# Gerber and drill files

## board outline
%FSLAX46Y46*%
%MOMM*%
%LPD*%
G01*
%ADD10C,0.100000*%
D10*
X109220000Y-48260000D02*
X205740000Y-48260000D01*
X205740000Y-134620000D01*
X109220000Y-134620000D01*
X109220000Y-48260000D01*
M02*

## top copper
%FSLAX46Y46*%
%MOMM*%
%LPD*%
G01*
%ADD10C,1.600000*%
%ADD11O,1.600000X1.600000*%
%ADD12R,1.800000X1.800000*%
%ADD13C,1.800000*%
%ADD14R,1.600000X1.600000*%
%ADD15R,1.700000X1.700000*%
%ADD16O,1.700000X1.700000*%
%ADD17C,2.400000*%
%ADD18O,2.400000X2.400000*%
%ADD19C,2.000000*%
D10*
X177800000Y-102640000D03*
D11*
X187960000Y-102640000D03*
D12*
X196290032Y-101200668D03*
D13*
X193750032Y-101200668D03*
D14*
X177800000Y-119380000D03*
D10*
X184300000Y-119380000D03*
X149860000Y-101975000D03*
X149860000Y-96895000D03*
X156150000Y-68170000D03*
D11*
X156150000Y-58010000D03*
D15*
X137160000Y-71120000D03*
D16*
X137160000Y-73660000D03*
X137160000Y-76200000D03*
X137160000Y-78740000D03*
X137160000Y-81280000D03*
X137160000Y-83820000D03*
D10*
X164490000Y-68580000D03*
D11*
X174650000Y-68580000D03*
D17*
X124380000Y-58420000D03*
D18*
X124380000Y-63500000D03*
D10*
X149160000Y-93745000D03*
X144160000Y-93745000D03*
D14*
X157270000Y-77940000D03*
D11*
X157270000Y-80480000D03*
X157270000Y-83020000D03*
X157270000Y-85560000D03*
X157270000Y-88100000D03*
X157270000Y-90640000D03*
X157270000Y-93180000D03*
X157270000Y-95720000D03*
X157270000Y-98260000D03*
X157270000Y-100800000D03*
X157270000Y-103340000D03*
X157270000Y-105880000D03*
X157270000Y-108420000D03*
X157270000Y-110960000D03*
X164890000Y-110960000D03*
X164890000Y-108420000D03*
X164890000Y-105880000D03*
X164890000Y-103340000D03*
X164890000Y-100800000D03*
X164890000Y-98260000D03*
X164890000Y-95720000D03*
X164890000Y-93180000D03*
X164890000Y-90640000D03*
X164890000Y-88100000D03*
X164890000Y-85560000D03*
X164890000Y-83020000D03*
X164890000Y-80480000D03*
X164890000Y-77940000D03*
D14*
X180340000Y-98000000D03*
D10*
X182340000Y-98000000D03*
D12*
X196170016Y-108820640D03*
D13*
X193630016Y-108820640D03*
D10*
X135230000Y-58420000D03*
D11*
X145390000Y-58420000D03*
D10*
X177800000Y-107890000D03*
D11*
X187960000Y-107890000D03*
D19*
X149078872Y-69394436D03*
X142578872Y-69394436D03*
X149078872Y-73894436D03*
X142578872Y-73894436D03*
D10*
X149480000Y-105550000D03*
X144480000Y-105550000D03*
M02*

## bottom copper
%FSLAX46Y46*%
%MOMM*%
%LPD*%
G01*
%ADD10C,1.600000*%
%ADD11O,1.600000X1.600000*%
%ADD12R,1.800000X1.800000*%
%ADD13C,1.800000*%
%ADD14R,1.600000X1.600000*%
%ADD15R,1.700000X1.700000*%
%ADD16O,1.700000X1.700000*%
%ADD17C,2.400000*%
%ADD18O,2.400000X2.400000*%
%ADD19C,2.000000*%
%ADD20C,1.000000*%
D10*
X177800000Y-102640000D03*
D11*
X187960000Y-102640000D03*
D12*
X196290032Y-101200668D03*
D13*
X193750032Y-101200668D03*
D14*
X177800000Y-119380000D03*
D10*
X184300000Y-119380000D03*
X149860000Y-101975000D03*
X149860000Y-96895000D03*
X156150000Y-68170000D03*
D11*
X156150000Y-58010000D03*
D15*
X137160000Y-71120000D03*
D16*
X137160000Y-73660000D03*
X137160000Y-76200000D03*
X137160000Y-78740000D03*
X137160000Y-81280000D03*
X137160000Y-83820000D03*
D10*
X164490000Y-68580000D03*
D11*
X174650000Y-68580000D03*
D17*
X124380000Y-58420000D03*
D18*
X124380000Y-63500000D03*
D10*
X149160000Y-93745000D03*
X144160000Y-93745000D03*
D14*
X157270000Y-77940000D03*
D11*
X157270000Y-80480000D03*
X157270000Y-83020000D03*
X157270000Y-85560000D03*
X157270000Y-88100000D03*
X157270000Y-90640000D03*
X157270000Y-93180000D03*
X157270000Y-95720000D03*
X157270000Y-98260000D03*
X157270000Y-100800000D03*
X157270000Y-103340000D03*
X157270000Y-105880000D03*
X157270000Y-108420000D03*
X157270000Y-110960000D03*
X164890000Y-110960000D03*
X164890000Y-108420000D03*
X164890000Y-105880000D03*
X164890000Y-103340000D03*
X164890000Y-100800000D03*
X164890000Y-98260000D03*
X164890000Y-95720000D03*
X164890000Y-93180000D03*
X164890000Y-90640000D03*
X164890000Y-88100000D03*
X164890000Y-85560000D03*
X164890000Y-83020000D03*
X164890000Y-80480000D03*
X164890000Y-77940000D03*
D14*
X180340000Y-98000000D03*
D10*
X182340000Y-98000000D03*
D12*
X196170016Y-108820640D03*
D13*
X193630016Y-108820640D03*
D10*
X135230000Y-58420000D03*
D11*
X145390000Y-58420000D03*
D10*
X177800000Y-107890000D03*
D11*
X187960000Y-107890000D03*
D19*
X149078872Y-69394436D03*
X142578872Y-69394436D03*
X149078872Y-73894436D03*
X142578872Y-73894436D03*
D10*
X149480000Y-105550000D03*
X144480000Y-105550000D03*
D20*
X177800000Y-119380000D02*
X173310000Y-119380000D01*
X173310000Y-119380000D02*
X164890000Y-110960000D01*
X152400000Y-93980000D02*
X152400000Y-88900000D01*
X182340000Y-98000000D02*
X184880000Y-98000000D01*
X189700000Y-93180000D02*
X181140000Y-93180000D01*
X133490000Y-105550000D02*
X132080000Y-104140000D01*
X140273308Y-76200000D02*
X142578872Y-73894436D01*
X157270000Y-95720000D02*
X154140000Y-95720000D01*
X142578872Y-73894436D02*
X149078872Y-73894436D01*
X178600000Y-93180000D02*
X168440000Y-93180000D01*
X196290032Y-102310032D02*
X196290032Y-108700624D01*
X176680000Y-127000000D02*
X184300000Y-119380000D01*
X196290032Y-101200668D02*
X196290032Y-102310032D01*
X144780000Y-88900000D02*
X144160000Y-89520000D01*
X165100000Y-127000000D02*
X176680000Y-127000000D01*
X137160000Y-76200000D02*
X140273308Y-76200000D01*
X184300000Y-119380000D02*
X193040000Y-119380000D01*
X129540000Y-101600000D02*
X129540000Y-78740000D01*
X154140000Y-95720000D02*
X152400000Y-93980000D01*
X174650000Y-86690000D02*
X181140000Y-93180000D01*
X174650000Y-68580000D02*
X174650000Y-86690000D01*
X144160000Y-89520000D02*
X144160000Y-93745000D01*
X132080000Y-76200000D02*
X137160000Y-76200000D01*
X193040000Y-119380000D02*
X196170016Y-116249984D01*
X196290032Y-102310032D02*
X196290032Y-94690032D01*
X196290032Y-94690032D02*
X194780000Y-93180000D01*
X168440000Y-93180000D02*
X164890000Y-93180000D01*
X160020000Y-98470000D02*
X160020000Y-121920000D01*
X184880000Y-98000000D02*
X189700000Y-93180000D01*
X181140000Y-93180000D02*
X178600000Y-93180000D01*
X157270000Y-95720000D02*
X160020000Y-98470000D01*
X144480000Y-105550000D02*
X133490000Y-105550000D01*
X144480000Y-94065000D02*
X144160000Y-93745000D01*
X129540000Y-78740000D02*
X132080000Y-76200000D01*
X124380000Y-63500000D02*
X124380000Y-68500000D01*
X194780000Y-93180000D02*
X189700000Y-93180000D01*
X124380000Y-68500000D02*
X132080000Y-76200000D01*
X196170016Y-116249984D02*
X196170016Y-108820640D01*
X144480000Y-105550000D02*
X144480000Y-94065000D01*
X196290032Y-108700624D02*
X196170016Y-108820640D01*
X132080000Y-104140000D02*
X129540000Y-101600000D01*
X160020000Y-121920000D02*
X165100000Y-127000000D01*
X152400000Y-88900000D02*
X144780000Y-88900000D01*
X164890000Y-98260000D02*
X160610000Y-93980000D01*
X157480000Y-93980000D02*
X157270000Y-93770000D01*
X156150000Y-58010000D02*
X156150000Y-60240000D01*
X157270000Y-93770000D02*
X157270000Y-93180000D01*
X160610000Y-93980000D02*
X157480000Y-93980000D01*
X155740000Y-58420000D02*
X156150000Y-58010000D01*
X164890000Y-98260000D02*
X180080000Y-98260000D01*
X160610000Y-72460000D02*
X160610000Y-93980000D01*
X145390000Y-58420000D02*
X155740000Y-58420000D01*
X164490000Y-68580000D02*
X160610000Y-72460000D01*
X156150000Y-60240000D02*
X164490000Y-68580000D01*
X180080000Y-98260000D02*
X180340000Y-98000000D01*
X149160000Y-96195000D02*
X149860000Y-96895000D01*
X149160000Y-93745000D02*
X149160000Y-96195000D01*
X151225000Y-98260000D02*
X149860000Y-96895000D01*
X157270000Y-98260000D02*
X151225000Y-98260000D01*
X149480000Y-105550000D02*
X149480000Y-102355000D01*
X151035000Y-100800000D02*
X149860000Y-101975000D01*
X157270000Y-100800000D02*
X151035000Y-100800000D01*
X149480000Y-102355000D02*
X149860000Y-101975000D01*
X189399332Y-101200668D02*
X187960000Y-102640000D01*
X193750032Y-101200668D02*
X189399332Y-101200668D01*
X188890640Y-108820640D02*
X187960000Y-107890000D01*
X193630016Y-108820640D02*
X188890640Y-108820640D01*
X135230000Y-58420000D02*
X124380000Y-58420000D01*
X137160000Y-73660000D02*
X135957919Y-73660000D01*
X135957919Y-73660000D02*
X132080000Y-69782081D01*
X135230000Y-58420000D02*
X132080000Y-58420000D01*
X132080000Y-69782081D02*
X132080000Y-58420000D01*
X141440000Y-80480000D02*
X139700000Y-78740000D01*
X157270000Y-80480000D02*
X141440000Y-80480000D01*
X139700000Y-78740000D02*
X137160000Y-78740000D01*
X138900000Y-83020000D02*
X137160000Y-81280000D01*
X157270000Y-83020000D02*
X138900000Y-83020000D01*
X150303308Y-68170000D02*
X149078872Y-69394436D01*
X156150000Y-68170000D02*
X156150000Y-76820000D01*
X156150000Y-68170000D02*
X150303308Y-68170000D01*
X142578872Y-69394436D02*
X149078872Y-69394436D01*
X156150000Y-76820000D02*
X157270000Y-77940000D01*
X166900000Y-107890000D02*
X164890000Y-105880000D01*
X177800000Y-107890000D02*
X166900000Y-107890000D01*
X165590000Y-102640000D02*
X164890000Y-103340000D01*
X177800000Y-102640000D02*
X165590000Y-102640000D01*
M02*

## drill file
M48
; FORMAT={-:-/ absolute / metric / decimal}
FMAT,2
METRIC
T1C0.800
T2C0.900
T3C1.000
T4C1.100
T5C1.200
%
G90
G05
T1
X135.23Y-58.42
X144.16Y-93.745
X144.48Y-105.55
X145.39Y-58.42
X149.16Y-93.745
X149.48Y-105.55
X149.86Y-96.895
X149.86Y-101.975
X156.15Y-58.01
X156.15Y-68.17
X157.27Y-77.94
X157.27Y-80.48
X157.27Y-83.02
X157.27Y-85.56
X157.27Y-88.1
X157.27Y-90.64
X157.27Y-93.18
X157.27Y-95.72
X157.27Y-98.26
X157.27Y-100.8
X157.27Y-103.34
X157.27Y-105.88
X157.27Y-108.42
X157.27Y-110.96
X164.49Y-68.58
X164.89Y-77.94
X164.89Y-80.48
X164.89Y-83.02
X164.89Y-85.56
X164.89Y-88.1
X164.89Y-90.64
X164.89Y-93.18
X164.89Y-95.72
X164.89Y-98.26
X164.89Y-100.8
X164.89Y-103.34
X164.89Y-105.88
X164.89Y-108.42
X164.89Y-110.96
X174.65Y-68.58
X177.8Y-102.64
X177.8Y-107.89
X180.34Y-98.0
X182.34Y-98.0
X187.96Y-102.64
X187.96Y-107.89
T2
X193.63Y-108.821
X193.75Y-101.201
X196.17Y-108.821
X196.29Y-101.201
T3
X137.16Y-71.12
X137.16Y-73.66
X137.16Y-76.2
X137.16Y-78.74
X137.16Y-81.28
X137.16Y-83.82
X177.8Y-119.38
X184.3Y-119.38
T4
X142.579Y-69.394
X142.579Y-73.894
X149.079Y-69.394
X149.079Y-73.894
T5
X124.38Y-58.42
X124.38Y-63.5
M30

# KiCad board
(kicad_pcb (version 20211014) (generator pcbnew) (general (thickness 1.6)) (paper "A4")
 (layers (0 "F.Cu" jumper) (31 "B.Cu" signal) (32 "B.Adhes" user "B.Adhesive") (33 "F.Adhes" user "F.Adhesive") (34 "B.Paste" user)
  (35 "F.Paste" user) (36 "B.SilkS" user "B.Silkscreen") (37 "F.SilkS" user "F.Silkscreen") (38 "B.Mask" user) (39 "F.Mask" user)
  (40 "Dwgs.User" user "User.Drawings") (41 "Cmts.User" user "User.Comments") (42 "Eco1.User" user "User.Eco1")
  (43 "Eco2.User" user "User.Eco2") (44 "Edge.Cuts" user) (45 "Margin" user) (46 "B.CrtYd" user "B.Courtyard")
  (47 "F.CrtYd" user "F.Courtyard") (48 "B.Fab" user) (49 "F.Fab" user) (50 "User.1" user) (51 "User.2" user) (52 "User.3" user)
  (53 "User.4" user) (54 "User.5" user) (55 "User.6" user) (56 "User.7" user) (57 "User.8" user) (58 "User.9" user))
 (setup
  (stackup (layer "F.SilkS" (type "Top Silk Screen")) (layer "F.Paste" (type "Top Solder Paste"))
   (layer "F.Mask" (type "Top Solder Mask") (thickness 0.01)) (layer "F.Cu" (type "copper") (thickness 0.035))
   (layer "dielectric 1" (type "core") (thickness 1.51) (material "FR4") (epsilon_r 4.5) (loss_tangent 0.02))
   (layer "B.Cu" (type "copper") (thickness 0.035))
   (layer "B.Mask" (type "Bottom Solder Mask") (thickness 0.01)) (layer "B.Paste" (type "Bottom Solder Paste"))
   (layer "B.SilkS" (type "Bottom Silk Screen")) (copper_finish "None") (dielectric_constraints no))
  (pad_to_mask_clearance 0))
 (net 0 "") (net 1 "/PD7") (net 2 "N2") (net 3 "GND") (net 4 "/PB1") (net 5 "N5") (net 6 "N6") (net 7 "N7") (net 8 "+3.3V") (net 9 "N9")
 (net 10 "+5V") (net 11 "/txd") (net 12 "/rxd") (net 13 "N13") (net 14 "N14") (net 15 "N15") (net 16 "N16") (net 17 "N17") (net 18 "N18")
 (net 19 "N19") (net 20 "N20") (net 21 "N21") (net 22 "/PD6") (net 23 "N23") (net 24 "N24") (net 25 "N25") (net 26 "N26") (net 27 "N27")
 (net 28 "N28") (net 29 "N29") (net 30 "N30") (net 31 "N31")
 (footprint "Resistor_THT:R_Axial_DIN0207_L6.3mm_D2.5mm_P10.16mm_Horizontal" (layer "F.Cu") (at 177.8 102.64)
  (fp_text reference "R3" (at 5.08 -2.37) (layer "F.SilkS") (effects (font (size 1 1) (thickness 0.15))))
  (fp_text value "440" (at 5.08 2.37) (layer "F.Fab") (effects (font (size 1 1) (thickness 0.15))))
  (pad "1" thru_hole circle (at 0 0) (size 1.6 1.6) (drill 0.8) (layers *.Cu *.Mask) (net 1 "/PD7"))
  (pad "2" thru_hole oval (at 10.16 0) (size 1.6 1.6) (drill 0.8) (layers *.Cu *.Mask) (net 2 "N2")))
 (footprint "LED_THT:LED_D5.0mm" (layer "F.Cu") (at 196.290032 101.200668 180)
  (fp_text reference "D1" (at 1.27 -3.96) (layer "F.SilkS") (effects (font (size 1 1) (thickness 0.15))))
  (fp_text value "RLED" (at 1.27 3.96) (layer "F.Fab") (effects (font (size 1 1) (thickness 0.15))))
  (pad "1" thru_hole rect (at 0 0 180) (size 1.8 1.8) (drill 0.9) (layers *.Cu *.Mask) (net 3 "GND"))
  (pad "2" thru_hole circle (at 2.54 0 180) (size 1.8 1.8) (drill 0.9) (layers *.Cu *.Mask) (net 2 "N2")))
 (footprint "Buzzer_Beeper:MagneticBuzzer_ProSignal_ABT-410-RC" (layer "F.Cu") (at 177.8 119.38)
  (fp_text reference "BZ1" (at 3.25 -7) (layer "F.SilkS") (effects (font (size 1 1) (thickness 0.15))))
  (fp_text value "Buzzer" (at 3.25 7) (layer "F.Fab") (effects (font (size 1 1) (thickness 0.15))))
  (pad "1" thru_hole rect (at 0 0) (size 1.6 1.6) (drill 1) (layers *.Cu *.Mask) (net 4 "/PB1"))
  (pad "2" thru_hole circle (at 6.5 0) (size 1.6 1.6) (drill 1) (layers *.Cu *.Mask) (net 3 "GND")))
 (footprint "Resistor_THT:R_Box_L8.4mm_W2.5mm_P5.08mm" (layer "F.Cu") (at 149.86 101.975 90)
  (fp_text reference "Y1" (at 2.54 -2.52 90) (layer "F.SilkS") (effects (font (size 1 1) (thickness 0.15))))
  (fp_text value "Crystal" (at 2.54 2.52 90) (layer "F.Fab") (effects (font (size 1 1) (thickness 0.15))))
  (pad "1" thru_hole circle (at 0 0 90) (size 1.6 1.6) (drill 0.8) (layers *.Cu *.Mask) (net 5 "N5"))
  (pad "2" thru_hole circle (at 5.08 0 90) (size 1.6 1.6) (drill 0.8) (layers *.Cu *.Mask) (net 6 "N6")))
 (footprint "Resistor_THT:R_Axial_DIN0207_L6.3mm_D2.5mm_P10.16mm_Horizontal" (layer "F.Cu") (at 156.15 68.17 90)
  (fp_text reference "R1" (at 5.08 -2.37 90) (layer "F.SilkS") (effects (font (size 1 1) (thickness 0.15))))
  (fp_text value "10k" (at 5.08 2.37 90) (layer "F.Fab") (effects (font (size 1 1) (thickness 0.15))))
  (pad "1" thru_hole circle (at 0 0 90) (size 1.6 1.6) (drill 0.8) (layers *.Cu *.Mask) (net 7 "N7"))
  (pad "2" thru_hole oval (at 10.16 0 90) (size 1.6 1.6) (drill 0.8) (layers *.Cu *.Mask) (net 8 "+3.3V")))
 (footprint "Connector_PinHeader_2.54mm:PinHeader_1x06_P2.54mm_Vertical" (layer "F.Cu") (at 137.16 71.12)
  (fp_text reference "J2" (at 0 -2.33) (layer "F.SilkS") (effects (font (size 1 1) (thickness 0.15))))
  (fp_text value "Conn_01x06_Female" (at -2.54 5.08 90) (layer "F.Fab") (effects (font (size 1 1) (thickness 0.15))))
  (pad "1" thru_hole rect (at 0 0) (size 1.7 1.7) (drill 1) (layers *.Cu *.Mask) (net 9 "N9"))
  (pad "2" thru_hole oval (at 0 2.54) (size 1.7 1.7) (drill 1) (layers *.Cu *.Mask) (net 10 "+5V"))
  (pad "3" thru_hole oval (at 0 5.08) (size 1.7 1.7) (drill 1) (layers *.Cu *.Mask) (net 3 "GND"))
  (pad "4" thru_hole oval (at 0 7.62) (size 1.7 1.7) (drill 1) (layers *.Cu *.Mask) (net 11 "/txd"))
  (pad "5" thru_hole oval (at 0 10.16) (size 1.7 1.7) (drill 1) (layers *.Cu *.Mask) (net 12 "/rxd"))
  (pad "6" thru_hole oval (at 0 12.7) (size 1.7 1.7) (drill 1) (layers *.Cu *.Mask) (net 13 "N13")))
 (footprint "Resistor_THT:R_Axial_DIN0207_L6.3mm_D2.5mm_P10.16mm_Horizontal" (layer "F.Cu") (at 164.49 68.58)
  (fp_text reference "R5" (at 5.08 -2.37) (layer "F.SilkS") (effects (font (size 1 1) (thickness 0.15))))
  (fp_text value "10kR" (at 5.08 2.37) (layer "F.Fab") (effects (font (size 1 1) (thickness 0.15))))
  (pad "1" thru_hole circle (at 0 0) (size 1.6 1.6) (drill 0.8) (layers *.Cu *.Mask) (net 8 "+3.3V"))
  (pad "2" thru_hole oval (at 10.16 0) (size 1.6 1.6) (drill 0.8) (layers *.Cu *.Mask) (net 3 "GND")))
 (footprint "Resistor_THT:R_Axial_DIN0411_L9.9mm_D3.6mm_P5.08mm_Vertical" (layer "F.Cu") (at 124.38 58.42 -90)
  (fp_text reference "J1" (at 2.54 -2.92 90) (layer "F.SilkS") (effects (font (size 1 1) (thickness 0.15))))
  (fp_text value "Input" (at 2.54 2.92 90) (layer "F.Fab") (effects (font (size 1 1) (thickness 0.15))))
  (pad "1" thru_hole circle (at 0 0 270) (size 2.4 2.4) (drill 1.2) (layers *.Cu *.Mask) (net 10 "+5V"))
  (pad "2" thru_hole oval (at 5.08 0 270) (size 2.4 2.4) (drill 1.2) (layers *.Cu *.Mask) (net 3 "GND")))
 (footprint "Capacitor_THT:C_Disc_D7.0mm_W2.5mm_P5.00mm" (layer "F.Cu") (at 149.16 93.745 180)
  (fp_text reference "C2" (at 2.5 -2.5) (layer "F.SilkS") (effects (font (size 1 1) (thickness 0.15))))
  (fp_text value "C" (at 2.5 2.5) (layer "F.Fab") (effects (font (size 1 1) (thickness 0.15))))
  (pad "1" thru_hole circle (at 0 0 180) (size 1.6 1.6) (drill 0.8) (layers *.Cu *.Mask) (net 6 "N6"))
  (pad "2" thru_hole circle (at 5 0 180) (size 1.6 1.6) (drill 0.8) (layers *.Cu *.Mask) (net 3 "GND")))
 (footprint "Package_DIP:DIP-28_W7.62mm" (layer "F.Cu") (at 157.27 77.94)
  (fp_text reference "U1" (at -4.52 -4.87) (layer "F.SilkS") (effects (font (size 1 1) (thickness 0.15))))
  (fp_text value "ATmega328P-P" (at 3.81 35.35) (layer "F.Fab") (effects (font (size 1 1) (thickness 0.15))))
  (pad "1" thru_hole rect (at 0 0) (size 1.6 1.6) (drill 0.8) (layers *.Cu *.Mask) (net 7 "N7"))
  (pad "2" thru_hole oval (at 0 2.54) (size 1.6 1.6) (drill 0.8) (layers *.Cu *.Mask) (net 11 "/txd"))
  (pad "3" thru_hole oval (at 0 5.08) (size 1.6 1.6) (drill 0.8) (layers *.Cu *.Mask) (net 12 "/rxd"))
  (pad "4" thru_hole oval (at 0 7.62) (size 1.6 1.6) (drill 0.8) (layers *.Cu *.Mask) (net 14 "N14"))
  (pad "5" thru_hole oval (at 0 10.16) (size 1.6 1.6) (drill 0.8) (layers *.Cu *.Mask) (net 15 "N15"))
  (pad "6" thru_hole oval (at 0 12.7) (size 1.6 1.6) (drill 0.8) (layers *.Cu *.Mask) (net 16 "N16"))
  (pad "7" thru_hole oval (at 0 15.24) (size 1.6 1.6) (drill 0.8) (layers *.Cu *.Mask) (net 8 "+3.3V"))
  (pad "8" thru_hole oval (at 0 17.78) (size 1.6 1.6) (drill 0.8) (layers *.Cu *.Mask) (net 3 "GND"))
  (pad "9" thru_hole oval (at 0 20.32) (size 1.6 1.6) (drill 0.8) (layers *.Cu *.Mask) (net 6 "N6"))
  (pad "10" thru_hole oval (at 0 22.86) (size 1.6 1.6) (drill 0.8) (layers *.Cu *.Mask) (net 5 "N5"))
  (pad "11" thru_hole oval (at 0 25.4) (size 1.6 1.6) (drill 0.8) (layers *.Cu *.Mask) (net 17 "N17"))
  (pad "12" thru_hole oval (at 0 27.94) (size 1.6 1.6) (drill 0.8) (layers *.Cu *.Mask) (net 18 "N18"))
  (pad "13" thru_hole oval (at 0 30.48) (size 1.6 1.6) (drill 0.8) (layers *.Cu *.Mask) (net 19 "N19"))
  (pad "14" thru_hole oval (at 0 33.02) (size 1.6 1.6) (drill 0.8) (layers *.Cu *.Mask) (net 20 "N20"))
  (pad "15" thru_hole oval (at 7.62 33.02) (size 1.6 1.6) (drill 0.8) (layers *.Cu *.Mask) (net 4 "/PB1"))
  (pad "16" thru_hole oval (at 7.62 30.48) (size 1.6 1.6) (drill 0.8) (layers *.Cu *.Mask) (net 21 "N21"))
  (pad "17" thru_hole oval (at 7.62 27.94) (size 1.6 1.6) (drill 0.8) (layers *.Cu *.Mask) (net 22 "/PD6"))
  (pad "18" thru_hole oval (at 7.62 25.4) (size 1.6 1.6) (drill 0.8) (layers *.Cu *.Mask) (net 1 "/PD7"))
  (pad "19" thru_hole oval (at 7.62 22.86) (size 1.6 1.6) (drill 0.8) (layers *.Cu *.Mask) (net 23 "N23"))
  (pad "20" thru_hole oval (at 7.62 20.32) (size 1.6 1.6) (drill 0.8) (layers *.Cu *.Mask) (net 8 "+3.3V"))
  (pad "21" thru_hole oval (at 7.62 17.78) (size 1.6 1.6) (drill 0.8) (layers *.Cu *.Mask) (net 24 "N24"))
  (pad "22" thru_hole oval (at 7.62 15.24) (size 1.6 1.6) (drill 0.8) (layers *.Cu *.Mask) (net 3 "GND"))
  (pad "23" thru_hole oval (at 7.62 12.7) (size 1.6 1.6) (drill 0.8) (layers *.Cu *.Mask) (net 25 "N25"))
  (pad "24" thru_hole oval (at 7.62 10.16) (size 1.6 1.6) (drill 0.8) (layers *.Cu *.Mask) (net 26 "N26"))
  (pad "25" thru_hole oval (at 7.62 7.62) (size 1.6 1.6) (drill 0.8) (layers *.Cu *.Mask) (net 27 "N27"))
  (pad "26" thru_hole oval (at 7.62 5.08) (size 1.6 1.6) (drill 0.8) (layers *.Cu *.Mask) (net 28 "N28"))
  (pad "27" thru_hole oval (at 7.62 2.54) (size 1.6 1.6) (drill 0.8) (layers *.Cu *.Mask) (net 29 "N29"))
  (pad "28" thru_hole oval (at 7.62 0) (size 1.6 1.6) (drill 0.8) (layers *.Cu *.Mask) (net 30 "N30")))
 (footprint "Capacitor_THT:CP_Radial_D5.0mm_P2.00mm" (layer "F.Cu") (at 180.34 98)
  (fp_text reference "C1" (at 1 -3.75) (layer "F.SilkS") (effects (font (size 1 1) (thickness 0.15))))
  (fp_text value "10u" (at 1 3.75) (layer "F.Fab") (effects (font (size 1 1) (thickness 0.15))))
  (pad "1" thru_hole rect (at 0 0) (size 1.6 1.6) (drill 0.8) (layers *.Cu *.Mask) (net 8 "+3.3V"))
  (pad "2" thru_hole circle (at 2 0) (size 1.6 1.6) (drill 0.8) (layers *.Cu *.Mask) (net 3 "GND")))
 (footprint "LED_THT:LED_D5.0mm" (layer "F.Cu") (at 196.170016 108.82064 180)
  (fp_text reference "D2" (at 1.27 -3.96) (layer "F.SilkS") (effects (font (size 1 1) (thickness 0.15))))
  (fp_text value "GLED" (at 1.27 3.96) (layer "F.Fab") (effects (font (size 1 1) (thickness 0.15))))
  (pad "1" thru_hole rect (at 0 0 180) (size 1.8 1.8) (drill 0.9) (layers *.Cu *.Mask) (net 3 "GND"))
  (pad "2" thru_hole circle (at 2.54 0 180) (size 1.8 1.8) (drill 0.9) (layers *.Cu *.Mask) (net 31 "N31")))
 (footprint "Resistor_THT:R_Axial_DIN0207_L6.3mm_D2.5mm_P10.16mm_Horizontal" (layer "F.Cu") (at 135.23 58.42)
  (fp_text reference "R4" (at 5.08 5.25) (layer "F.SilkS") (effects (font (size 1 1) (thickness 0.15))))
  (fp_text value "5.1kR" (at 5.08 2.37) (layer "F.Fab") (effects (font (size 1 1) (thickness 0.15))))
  (pad "1" thru_hole circle (at 0 0) (size 1.6 1.6) (drill 0.8) (layers *.Cu *.Mask) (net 10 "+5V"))
  (pad "2" thru_hole oval (at 10.16 0) (size 1.6 1.6) (drill 0.8) (layers *.Cu *.Mask) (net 8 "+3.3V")))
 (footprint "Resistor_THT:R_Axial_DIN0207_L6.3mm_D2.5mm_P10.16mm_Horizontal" (layer "F.Cu") (at 177.8 107.89)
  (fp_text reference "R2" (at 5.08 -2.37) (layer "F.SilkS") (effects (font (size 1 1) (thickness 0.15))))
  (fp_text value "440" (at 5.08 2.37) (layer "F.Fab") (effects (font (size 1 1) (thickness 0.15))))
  (pad "1" thru_hole circle (at 0 0) (size 1.6 1.6) (drill 0.8) (layers *.Cu *.Mask) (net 22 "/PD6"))
  (pad "2" thru_hole oval (at 10.16 0) (size 1.6 1.6) (drill 0.8) (layers *.Cu *.Mask) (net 31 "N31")))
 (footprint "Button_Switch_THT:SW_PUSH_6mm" (layer "F.Cu") (at 142.578872 69.394436)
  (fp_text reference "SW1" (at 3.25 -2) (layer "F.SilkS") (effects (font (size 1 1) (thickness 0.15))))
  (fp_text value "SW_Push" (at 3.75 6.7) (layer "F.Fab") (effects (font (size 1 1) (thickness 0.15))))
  (pad "1" thru_hole circle (at 6.5 0 90) (size 2 2) (drill 1.1) (layers *.Cu *.Mask) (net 7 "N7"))
  (pad "1" thru_hole circle (at 0 0 90) (size 2 2) (drill 1.1) (layers *.Cu *.Mask) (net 7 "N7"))
  (pad "2" thru_hole circle (at 6.5 4.5 90) (size 2 2) (drill 1.1) (layers *.Cu *.Mask) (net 3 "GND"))
  (pad "2" thru_hole circle (at 0 4.5 90) (size 2 2) (drill 1.1) (layers *.Cu *.Mask) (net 3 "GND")))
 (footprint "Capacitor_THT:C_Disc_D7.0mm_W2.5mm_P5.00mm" (layer "F.Cu") (at 149.48 105.55 180)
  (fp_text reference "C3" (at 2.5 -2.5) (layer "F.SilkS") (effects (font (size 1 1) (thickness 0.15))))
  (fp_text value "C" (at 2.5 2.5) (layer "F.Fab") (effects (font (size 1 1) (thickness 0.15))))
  (pad "1" thru_hole circle (at 0 0 180) (size 1.6 1.6) (drill 0.8) (layers *.Cu *.Mask) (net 5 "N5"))
  (pad "2" thru_hole circle (at 5 0 180) (size 1.6 1.6) (drill 0.8) (layers *.Cu *.Mask) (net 3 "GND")))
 (gr_rect (start 205.74 134.62) (end 109.22 48.26) (layer "Edge.Cuts") (width 0.1) (fill none))
 (segment (start 177.8 119.38) (end 173.31 119.38) (width 1) (layer "B.Cu") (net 4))
 (segment (start 173.31 119.38) (end 164.89 110.96) (width 1) (layer "B.Cu") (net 4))
 (segment (start 152.4 93.98) (end 152.4 88.9) (width 1) (layer "B.Cu") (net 3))
 (segment (start 182.34 98) (end 184.88 98) (width 1) (layer "B.Cu") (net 3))
 (segment (start 189.7 93.18) (end 181.14 93.18) (width 1) (layer "B.Cu") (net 3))
 (segment (start 133.49 105.55) (end 132.08 104.14) (width 1) (layer "B.Cu") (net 3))
 (segment (start 140.273308 76.2) (end 142.578872 73.894436) (width 1) (layer "B.Cu") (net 3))
 (segment (start 157.27 95.72) (end 154.14 95.72) (width 1) (layer "B.Cu") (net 3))
 (segment (start 142.578872 73.894436) (end 149.078872 73.894436) (width 1) (layer "B.Cu") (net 3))
 (segment (start 178.6 93.18) (end 168.44 93.18) (width 1) (layer "B.Cu") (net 3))
 (segment (start 196.290032 102.310032) (end 196.290032 108.700624) (width 1) (layer "B.Cu") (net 3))
 (segment (start 176.68 127) (end 184.3 119.38) (width 1) (layer "B.Cu") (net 3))
 (segment (start 196.290032 101.200668) (end 196.290032 102.310032) (width 1) (layer "B.Cu") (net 3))
 (segment (start 144.78 88.9) (end 144.16 89.52) (width 1) (layer "B.Cu") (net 3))
 (segment (start 165.1 127) (end 176.68 127) (width 1) (layer "B.Cu") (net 3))
 (segment (start 137.16 76.2) (end 140.273308 76.2) (width 1) (layer "B.Cu") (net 3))
 (segment (start 184.3 119.38) (end 193.04 119.38) (width 1) (layer "B.Cu") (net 3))
 (segment (start 129.54 101.6) (end 129.54 78.74) (width 1) (layer "B.Cu") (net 3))
 (segment (start 154.14 95.72) (end 152.4 93.98) (width 1) (layer "B.Cu") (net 3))
 (segment (start 174.65 86.69) (end 181.14 93.18) (width 1) (layer "B.Cu") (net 3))
 (segment (start 174.65 68.58) (end 174.65 86.69) (width 1) (layer "B.Cu") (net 3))
 (segment (start 144.16 89.52) (end 144.16 93.745) (width 1) (layer "B.Cu") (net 3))
 (segment (start 132.08 76.2) (end 137.16 76.2) (width 1) (layer "B.Cu") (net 3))
 (segment (start 193.04 119.38) (end 196.170016 116.249984) (width 1) (layer "B.Cu") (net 3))
 (segment (start 196.290032 102.310032) (end 196.290032 94.690032) (width 1) (layer "B.Cu") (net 3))
 (segment (start 196.290032 94.690032) (end 194.78 93.18) (width 1) (layer "B.Cu") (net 3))
 (segment (start 168.44 93.18) (end 164.89 93.18) (width 1) (layer "B.Cu") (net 3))
 (segment (start 160.02 98.47) (end 160.02 121.92) (width 1) (layer "B.Cu") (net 3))
 (segment (start 184.88 98) (end 189.7 93.18) (width 1) (layer "B.Cu") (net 3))
 (segment (start 181.14 93.18) (end 178.6 93.18) (width 1) (layer "B.Cu") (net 3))
 (segment (start 157.27 95.72) (end 160.02 98.47) (width 1) (layer "B.Cu") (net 3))
 (segment (start 144.48 105.55) (end 133.49 105.55) (width 1) (layer "B.Cu") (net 3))
 (segment (start 144.48 94.065) (end 144.16 93.745) (width 1) (layer "B.Cu") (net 3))
 (segment (start 129.54 78.74) (end 132.08 76.2) (width 1) (layer "B.Cu") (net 3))
 (segment (start 124.38 63.5) (end 124.38 68.5) (width 1) (layer "B.Cu") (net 3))
 (segment (start 194.78 93.18) (end 189.7 93.18) (width 1) (layer "B.Cu") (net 3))
 (segment (start 124.38 68.5) (end 132.08 76.2) (width 1) (layer "B.Cu") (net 3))
 (segment (start 196.170016 116.249984) (end 196.170016 108.82064) (width 1) (layer "B.Cu") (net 3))
 (segment (start 144.48 105.55) (end 144.48 94.065) (width 1) (layer "B.Cu") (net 3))
 (segment (start 196.290032 108.700624) (end 196.170016 108.82064) (width 1) (layer "B.Cu") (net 3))
 (segment (start 132.08 104.14) (end 129.54 101.6) (width 1) (layer "B.Cu") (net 3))
 (segment (start 160.02 121.92) (end 165.1 127) (width 1) (layer "B.Cu") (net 3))
 (segment (start 152.4 88.9) (end 144.78 88.9) (width 1) (layer "B.Cu") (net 3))
 (segment (start 164.89 98.26) (end 160.61 93.98) (width 1) (layer "B.Cu") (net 8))
 (segment (start 157.48 93.98) (end 157.27 93.77) (width 1) (layer "B.Cu") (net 8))
 (segment (start 156.15 58.01) (end 156.15 60.24) (width 1) (layer "B.Cu") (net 8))
 (segment (start 157.27 93.77) (end 157.27 93.18) (width 1) (layer "B.Cu") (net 8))
 (segment (start 160.61 93.98) (end 157.48 93.98) (width 1) (layer "B.Cu") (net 8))
 (segment (start 155.74 58.42) (end 156.15 58.01) (width 1) (layer "B.Cu") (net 8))
 (segment (start 164.89 98.26) (end 180.08 98.26) (width 1) (layer "B.Cu") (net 8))
 (segment (start 160.61 72.46) (end 160.61 93.98) (width 1) (layer "B.Cu") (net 8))
 (segment (start 145.39 58.42) (end 155.74 58.42) (width 1) (layer "B.Cu") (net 8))
 (segment (start 164.49 68.58) (end 160.61 72.46) (width 1) (layer "B.Cu") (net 8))
 (segment (start 156.15 60.24) (end 164.49 68.58) (width 1) (layer "B.Cu") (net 8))
 (segment (start 180.08 98.26) (end 180.34 98) (width 1) (layer "B.Cu") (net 8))
 (segment (start 149.16 96.195) (end 149.86 96.895) (width 1) (layer "B.Cu") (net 6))
 (segment (start 149.16 93.745) (end 149.16 96.195) (width 1) (layer "B.Cu") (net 6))
 (segment (start 151.225 98.26) (end 149.86 96.895) (width 1) (layer "B.Cu") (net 6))
 (segment (start 157.27 98.26) (end 151.225 98.26) (width 1) (layer "B.Cu") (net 6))
 (segment (start 149.48 105.55) (end 149.48 102.355) (width 1) (layer "B.Cu") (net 5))
 (segment (start 151.035 100.8) (end 149.86 101.975) (width 1) (layer "B.Cu") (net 5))
 (segment (start 157.27 100.8) (end 151.035 100.8) (width 1) (layer "B.Cu") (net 5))
 (segment (start 149.48 102.355) (end 149.86 101.975) (width 1) (layer "B.Cu") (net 5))
 (segment (start 189.399332 101.200668) (end 187.96 102.64) (width 1) (layer "B.Cu") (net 2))
 (segment (start 193.750032 101.200668) (end 189.399332 101.200668) (width 1) (layer "B.Cu") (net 2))
 (segment (start 188.89064 108.82064) (end 187.96 107.89) (width 1) (layer "B.Cu") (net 31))
 (segment (start 193.630016 108.82064) (end 188.89064 108.82064) (width 1) (layer "B.Cu") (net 31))
 (segment (start 135.23 58.42) (end 124.38 58.42) (width 1) (layer "B.Cu") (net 10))
 (segment (start 137.16 73.66) (end 135.957919 73.66) (width 1) (layer "B.Cu") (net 10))
 (segment (start 135.957919 73.66) (end 132.08 69.782081) (width 1) (layer "B.Cu") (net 10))
 (segment (start 135.23 58.42) (end 132.08 58.42) (width 1) (layer "B.Cu") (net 10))
 (segment (start 132.08 69.782081) (end 132.08 58.42) (width 1) (layer "B.Cu") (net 10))
 (segment (start 141.44 80.48) (end 139.7 78.74) (width 1) (layer "B.Cu") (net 11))
 (segment (start 157.27 80.48) (end 141.44 80.48) (width 1) (layer "B.Cu") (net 11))
 (segment (start 139.7 78.74) (end 137.16 78.74) (width 1) (layer "B.Cu") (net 11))
 (segment (start 138.9 83.02) (end 137.16 81.28) (width 1) (layer "B.Cu") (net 12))
 (segment (start 157.27 83.02) (end 138.9 83.02) (width 1) (layer "B.Cu") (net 12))
 (segment (start 150.303308 68.17) (end 149.078872 69.394436) (width 1) (layer "B.Cu") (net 7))
 (segment (start 156.15 68.17) (end 156.15 76.82) (width 1) (layer "B.Cu") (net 7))
 (segment (start 156.15 68.17) (end 150.303308 68.17) (width 1) (layer "B.Cu") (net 7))
 (segment (start 142.578872 69.394436) (end 149.078872 69.394436) (width 1) (layer "B.Cu") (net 7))
 (segment (start 156.15 76.82) (end 157.27 77.94) (width 1) (layer "B.Cu") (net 7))
 (segment (start 166.9 107.89) (end 164.89 105.88) (width 1) (layer "B.Cu") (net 22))
 (segment (start 177.8 107.89) (end 166.9 107.89) (width 1) (layer "B.Cu") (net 22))
 (segment (start 165.59 102.64) (end 164.89 103.34) (width 1) (layer "B.Cu") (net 1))
 (segment (start 177.8 102.64) (end 165.59 102.64) (width 1) (layer "B.Cu") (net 1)))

